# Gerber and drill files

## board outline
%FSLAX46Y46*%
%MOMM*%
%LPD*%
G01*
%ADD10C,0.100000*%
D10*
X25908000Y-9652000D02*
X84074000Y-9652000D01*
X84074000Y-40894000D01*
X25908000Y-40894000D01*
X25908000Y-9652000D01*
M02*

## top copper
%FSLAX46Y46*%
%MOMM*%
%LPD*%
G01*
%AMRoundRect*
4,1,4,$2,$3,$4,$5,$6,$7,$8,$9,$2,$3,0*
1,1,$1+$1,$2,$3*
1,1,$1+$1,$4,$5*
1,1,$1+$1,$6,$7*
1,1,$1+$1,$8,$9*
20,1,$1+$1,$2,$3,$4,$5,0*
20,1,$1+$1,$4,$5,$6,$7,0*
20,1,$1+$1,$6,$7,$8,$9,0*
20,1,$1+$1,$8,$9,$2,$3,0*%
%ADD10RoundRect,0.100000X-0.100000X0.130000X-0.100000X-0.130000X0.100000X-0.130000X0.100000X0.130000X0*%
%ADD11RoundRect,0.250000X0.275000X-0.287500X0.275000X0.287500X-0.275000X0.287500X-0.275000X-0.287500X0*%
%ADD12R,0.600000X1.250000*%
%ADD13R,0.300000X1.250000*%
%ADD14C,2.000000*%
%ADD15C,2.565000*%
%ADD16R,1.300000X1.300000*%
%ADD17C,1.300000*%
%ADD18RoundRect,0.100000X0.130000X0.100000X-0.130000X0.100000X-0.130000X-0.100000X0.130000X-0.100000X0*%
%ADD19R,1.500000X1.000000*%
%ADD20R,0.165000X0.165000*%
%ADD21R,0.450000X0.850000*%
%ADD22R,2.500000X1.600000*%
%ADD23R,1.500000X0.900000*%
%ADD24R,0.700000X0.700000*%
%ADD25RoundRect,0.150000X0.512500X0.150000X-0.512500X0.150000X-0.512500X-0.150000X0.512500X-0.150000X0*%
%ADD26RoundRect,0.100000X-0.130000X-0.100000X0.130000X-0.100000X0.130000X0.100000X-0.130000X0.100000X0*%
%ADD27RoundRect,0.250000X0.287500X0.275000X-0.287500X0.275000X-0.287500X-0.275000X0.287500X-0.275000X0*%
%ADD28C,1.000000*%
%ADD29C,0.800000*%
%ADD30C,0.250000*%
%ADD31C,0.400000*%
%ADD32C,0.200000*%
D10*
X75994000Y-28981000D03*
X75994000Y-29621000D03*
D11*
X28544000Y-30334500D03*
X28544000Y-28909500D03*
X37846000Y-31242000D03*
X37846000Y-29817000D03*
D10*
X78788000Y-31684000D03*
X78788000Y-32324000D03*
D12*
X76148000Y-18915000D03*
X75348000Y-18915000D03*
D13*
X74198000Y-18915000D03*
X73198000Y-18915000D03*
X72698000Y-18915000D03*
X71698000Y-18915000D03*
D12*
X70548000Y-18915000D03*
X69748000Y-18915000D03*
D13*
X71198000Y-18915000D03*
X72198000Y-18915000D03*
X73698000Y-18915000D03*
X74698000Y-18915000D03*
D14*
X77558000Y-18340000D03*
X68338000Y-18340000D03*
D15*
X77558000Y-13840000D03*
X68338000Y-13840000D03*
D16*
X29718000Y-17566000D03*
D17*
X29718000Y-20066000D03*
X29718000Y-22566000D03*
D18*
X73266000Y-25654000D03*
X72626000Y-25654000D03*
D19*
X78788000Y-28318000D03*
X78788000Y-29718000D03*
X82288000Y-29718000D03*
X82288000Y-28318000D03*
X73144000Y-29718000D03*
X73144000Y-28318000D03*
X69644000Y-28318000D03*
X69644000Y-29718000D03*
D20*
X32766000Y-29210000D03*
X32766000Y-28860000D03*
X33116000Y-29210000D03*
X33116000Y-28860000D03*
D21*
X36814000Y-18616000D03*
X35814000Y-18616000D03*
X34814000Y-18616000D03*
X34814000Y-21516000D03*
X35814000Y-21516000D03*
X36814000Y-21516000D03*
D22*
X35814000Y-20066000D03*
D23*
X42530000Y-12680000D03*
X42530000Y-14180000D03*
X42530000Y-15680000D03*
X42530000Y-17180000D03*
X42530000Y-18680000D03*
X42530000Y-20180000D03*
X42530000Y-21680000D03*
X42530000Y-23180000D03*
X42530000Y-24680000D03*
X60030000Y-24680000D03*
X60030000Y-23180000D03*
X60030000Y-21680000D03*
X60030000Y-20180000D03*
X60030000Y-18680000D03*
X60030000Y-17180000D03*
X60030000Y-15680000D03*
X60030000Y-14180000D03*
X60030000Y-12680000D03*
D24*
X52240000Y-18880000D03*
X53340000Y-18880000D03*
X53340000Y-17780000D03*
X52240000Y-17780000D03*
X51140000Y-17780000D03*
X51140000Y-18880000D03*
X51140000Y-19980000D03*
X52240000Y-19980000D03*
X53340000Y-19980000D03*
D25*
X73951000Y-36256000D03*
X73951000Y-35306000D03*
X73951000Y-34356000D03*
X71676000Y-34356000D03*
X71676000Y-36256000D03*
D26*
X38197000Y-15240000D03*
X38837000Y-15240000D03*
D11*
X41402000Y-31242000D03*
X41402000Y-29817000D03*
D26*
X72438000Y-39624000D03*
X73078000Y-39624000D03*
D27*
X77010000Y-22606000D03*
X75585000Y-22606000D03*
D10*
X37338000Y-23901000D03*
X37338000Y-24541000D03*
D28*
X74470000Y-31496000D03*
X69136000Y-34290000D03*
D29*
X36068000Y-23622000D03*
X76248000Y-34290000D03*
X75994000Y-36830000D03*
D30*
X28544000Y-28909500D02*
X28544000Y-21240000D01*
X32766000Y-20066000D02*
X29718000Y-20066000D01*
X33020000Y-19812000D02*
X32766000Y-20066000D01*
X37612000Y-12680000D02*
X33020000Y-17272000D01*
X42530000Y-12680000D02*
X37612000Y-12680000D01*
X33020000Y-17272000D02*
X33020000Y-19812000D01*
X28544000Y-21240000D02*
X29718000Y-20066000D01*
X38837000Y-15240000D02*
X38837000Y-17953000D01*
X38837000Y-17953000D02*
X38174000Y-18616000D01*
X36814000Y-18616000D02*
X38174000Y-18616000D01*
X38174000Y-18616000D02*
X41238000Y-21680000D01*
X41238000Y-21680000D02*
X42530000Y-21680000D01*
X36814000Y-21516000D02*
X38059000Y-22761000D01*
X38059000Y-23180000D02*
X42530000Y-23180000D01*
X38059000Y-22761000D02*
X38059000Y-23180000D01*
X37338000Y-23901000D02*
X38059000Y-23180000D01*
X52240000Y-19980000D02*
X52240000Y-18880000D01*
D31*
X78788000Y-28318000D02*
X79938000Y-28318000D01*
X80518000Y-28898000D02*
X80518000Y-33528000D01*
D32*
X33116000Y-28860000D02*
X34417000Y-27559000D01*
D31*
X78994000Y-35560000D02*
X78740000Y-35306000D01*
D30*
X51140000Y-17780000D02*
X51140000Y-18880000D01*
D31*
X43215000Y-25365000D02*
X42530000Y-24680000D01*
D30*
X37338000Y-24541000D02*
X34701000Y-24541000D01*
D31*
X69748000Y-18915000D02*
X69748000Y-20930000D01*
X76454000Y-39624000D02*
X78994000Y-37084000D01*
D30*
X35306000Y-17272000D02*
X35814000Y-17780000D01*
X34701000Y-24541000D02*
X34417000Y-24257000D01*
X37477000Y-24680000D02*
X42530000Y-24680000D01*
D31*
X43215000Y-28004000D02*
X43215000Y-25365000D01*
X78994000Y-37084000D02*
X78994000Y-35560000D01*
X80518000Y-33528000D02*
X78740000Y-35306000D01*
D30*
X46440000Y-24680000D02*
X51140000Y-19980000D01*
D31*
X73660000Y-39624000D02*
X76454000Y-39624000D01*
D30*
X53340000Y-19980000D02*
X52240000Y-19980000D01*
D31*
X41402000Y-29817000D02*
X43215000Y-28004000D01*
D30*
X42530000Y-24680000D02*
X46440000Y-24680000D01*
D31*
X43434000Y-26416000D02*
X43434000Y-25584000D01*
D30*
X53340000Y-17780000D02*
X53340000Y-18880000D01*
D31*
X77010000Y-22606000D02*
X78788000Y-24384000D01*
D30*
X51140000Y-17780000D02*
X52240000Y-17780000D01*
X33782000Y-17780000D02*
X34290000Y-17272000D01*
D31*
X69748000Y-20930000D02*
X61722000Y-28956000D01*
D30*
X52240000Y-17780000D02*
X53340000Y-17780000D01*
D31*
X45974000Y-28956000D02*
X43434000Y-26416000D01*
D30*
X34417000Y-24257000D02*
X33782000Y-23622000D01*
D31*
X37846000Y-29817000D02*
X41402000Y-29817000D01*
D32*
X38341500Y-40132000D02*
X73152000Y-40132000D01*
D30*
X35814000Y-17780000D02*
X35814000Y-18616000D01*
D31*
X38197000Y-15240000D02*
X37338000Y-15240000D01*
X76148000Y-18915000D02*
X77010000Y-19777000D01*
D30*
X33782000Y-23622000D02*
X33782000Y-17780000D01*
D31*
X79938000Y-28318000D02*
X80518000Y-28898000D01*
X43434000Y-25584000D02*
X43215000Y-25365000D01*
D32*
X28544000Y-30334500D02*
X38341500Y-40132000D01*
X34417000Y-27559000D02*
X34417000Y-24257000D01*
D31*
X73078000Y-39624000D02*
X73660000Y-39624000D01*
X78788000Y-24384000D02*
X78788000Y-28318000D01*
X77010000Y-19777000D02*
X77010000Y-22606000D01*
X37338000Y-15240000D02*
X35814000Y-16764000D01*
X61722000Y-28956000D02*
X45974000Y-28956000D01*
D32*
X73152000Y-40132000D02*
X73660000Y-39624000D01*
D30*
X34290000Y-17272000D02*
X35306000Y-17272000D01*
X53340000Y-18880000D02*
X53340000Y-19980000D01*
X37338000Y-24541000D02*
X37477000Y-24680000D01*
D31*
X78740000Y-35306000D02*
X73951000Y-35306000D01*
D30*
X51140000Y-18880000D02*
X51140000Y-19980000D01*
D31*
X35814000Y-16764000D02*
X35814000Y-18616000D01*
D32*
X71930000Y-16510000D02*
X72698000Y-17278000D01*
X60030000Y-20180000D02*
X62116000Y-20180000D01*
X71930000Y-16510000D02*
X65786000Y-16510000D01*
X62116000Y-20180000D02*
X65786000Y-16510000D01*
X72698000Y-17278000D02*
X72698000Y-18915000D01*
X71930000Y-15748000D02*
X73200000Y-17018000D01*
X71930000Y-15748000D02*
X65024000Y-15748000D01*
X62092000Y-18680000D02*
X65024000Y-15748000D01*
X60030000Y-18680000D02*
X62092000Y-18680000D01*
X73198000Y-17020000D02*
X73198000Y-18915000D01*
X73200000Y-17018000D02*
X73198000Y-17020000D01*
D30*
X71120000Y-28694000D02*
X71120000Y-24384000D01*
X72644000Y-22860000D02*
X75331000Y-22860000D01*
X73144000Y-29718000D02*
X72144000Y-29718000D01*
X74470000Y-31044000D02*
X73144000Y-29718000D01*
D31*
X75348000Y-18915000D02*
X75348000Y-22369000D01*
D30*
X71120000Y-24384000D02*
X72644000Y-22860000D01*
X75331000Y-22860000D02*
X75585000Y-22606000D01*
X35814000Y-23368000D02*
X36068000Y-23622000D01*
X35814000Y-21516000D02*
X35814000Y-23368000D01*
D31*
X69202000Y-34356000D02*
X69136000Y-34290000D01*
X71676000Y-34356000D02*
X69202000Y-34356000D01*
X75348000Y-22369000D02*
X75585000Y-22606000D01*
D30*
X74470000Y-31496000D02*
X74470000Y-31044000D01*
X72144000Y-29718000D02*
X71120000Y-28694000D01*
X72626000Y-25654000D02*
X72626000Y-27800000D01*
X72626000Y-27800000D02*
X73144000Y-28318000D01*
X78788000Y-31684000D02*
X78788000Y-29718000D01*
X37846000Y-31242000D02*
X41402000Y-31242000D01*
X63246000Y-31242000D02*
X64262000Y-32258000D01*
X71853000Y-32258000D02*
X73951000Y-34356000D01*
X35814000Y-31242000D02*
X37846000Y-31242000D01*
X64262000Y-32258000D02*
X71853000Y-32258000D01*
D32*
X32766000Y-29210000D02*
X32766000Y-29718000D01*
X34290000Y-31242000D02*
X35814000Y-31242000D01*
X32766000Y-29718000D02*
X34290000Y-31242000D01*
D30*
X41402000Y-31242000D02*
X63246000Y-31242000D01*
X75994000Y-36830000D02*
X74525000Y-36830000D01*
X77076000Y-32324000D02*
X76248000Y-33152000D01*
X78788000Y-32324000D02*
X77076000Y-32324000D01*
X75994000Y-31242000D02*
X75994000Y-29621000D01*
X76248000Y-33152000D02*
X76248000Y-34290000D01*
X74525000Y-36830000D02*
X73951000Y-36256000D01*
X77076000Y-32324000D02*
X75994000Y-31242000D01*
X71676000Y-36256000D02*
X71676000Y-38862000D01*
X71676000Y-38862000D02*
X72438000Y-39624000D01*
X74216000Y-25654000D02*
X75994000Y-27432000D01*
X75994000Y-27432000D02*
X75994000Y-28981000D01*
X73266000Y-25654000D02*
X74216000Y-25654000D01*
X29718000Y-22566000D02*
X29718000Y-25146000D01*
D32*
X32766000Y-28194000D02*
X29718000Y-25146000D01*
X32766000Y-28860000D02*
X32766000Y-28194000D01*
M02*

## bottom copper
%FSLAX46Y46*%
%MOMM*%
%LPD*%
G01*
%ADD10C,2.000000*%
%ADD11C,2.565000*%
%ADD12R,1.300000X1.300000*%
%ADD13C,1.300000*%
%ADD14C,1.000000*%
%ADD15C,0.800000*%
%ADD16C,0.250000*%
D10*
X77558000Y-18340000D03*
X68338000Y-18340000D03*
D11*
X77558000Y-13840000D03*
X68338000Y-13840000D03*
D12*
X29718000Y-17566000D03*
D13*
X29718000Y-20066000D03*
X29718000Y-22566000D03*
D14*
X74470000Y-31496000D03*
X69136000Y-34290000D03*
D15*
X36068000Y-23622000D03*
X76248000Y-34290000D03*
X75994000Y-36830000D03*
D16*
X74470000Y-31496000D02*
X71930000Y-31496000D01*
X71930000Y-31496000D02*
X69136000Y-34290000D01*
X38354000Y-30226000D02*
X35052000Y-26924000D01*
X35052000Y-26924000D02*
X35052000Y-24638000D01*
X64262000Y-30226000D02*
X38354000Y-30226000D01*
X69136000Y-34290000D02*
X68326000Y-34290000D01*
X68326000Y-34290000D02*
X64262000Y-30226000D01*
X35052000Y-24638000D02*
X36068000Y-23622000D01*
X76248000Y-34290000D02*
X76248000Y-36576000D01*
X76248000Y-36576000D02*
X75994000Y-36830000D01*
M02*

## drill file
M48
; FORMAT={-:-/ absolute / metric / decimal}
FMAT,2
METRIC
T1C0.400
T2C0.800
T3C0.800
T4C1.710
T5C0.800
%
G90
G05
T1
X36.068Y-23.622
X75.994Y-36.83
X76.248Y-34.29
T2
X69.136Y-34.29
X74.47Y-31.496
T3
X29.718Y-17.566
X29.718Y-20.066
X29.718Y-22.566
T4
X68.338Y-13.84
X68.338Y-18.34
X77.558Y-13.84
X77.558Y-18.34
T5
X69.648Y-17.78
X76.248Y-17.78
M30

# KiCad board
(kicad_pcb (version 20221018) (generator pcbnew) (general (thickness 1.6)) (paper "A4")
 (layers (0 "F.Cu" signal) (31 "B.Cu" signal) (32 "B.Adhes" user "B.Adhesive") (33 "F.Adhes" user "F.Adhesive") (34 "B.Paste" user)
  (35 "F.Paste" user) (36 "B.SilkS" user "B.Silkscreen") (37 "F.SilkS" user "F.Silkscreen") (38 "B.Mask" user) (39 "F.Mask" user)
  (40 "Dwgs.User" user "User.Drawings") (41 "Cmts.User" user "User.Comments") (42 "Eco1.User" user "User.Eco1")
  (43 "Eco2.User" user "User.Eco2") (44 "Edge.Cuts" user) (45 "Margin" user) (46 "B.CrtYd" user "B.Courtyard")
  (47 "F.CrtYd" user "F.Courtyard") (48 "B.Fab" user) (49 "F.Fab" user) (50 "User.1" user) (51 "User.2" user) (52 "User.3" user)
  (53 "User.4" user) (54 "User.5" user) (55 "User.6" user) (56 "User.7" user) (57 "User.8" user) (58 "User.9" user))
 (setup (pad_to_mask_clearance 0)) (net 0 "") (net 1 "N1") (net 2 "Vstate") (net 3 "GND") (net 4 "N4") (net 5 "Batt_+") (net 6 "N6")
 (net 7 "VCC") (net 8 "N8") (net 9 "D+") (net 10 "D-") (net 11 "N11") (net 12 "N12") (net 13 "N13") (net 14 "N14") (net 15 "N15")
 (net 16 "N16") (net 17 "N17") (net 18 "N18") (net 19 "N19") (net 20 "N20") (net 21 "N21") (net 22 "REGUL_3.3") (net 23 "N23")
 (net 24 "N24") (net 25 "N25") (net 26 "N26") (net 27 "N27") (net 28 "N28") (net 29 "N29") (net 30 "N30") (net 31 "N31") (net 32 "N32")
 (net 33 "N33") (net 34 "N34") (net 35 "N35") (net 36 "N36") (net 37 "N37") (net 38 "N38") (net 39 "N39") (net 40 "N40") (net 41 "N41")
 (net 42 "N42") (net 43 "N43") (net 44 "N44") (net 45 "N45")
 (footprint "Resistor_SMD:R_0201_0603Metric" (layer "F.Cu") (at 75.994 29.301 -90)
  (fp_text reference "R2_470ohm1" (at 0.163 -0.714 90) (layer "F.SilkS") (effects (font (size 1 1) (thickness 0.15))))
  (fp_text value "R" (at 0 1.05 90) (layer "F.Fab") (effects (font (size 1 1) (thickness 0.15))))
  (pad "" smd roundrect (at -0.345 0 270) (size 0.318 0.36) (layers "F.Paste") (roundrect_rratio 0.25))
  (pad "" smd roundrect (at 0.345 0 270) (size 0.318 0.36) (layers "F.Paste") (roundrect_rratio 0.25))
  (pad "1" smd roundrect (at -0.32 0 270) (size 0.46 0.4) (layers "F.Cu" "F.Mask") (roundrect_rratio 0.25) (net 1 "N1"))
  (pad "2" smd roundrect (at 0.32 0 270) (size 0.46 0.4) (layers "F.Cu" "F.Mask") (roundrect_rratio 0.25) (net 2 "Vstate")))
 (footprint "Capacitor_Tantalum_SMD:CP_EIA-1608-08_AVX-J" (layer "F.Cu") (at 28.544 29.622 90)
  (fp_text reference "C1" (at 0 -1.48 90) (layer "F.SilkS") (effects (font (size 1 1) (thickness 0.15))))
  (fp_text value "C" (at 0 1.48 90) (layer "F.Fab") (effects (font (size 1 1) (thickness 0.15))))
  (pad "1" smd roundrect (at -0.7125 0 90) (size 1.075 1.05) (layers "F.Cu" "F.Paste" "F.Mask") (roundrect_rratio 0.238095) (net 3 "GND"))
  (pad "2" smd roundrect (at 0.7125 0 90) (size 1.075 1.05) (layers "F.Cu" "F.Paste" "F.Mask") (roundrect_rratio 0.238095) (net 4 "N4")))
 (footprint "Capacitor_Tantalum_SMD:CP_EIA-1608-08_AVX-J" (layer "F.Cu") (at 37.846 30.5295 90)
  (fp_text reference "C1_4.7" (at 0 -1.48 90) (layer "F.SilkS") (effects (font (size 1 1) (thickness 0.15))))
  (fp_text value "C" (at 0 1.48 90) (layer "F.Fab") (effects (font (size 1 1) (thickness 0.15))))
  (pad "1" smd roundrect (at -0.7125 0 90) (size 1.075 1.05) (layers "F.Cu" "F.Paste" "F.Mask") (roundrect_rratio 0.238095) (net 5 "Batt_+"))
  (pad "2" smd roundrect (at 0.7125 0 90) (size 1.075 1.05) (layers "F.Cu" "F.Paste" "F.Mask") (roundrect_rratio 0.238095) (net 3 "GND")))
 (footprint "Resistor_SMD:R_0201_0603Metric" (layer "F.Cu") (at 78.788 32.004 -90)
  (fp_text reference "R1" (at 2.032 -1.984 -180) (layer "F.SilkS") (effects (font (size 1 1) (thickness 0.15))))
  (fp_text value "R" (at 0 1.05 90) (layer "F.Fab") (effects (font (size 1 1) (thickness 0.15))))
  (pad "" smd roundrect (at -0.345 0 270) (size 0.318 0.36) (layers "F.Paste") (roundrect_rratio 0.25))
  (pad "" smd roundrect (at 0.345 0 270) (size 0.318 0.36) (layers "F.Paste") (roundrect_rratio 0.25))
  (pad "1" smd roundrect (at -0.32 0 270) (size 0.46 0.4) (layers "F.Cu" "F.Mask") (roundrect_rratio 0.25) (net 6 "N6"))
  (pad "2" smd roundrect (at 0.32 0 270) (size 0.46 0.4) (layers "F.Cu" "F.Mask") (roundrect_rratio 0.25) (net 2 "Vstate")))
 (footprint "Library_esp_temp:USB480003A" (layer "F.Cu") (at 72.948 15.24 180)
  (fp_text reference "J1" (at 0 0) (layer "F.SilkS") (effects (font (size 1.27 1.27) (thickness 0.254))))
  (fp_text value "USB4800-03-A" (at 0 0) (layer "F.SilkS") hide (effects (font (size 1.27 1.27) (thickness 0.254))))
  (pad "" np_thru_hole circle (at -3.3 -2.54 180) (size 0.8 0.8) (drill 0.8) (layers "*.Cu" "*.Mask"))
  (pad "" np_thru_hole circle (at 3.3 -2.54 180) (size 0.8 0.8) (drill 0.8) (layers "*.Cu" "*.Mask"))
  (pad "A1" smd rect (at -3.2 -3.675 180) (size 0.6 1.25) (layers "F.Cu" "F.Paste" "F.Mask") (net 3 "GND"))
  (pad "A4" smd rect (at -2.4 -3.675 180) (size 0.6 1.25) (layers "F.Cu" "F.Paste" "F.Mask") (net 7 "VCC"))
  (pad "A5" smd rect (at -1.25 -3.675 180) (size 0.3 1.25) (layers "F.Cu" "F.Paste" "F.Mask") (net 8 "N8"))
  (pad "A6" smd rect (at -0.25 -3.675 180) (size 0.3 1.25) (layers "F.Cu" "F.Paste" "F.Mask") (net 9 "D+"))
  (pad "A7" smd rect (at 0.25 -3.675 180) (size 0.3 1.25) (layers "F.Cu" "F.Paste" "F.Mask") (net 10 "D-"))
  (pad "A8" smd rect (at 1.25 -3.675 180) (size 0.3 1.25) (layers "F.Cu" "F.Paste" "F.Mask") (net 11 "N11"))
  (pad "A9" smd rect (at 2.4 -3.675 180) (size 0.6 1.25) (layers "F.Cu" "F.Paste" "F.Mask") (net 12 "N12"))
  (pad "A12" smd rect (at 3.2 -3.675 180) (size 0.6 1.25) (layers "F.Cu" "F.Paste" "F.Mask") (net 3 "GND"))
  (pad "B5" smd rect (at 1.75 -3.675 180) (size 0.3 1.25) (layers "F.Cu" "F.Paste" "F.Mask") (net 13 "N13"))
  (pad "B6" smd rect (at 0.75 -3.675 180) (size 0.3 1.25) (layers "F.Cu" "F.Paste" "F.Mask") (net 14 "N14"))
  (pad "B7" smd rect (at -0.75 -3.675 180) (size 0.3 1.25) (layers "F.Cu" "F.Paste" "F.Mask") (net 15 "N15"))
  (pad "B8" smd rect (at -1.75 -3.675 180) (size 0.3 1.25) (layers "F.Cu" "F.Paste" "F.Mask") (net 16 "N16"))
  (pad "MH3" thru_hole circle (at -4.61 -3.1 180) (size 2 2) (drill 1.71) (layers "*.Cu" "*.Mask") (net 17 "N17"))
  (pad "MH4" thru_hole circle (at 4.61 -3.1 180) (size 2 2) (drill 1.71) (layers "*.Cu" "*.Mask") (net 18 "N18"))
  (pad "MH5" thru_hole circle (at -4.61 1.4 180) (size 2.565 2.565) (drill 1.71) (layers "*.Cu" "*.Mask") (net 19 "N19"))
  (pad "MH6" thru_hole circle (at 4.61 1.4 180) (size 2.565 2.565) (drill 1.71) (layers "*.Cu" "*.Mask") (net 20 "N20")))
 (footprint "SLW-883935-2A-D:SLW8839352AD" (layer "F.Cu") (at 29.718 17.566 -90)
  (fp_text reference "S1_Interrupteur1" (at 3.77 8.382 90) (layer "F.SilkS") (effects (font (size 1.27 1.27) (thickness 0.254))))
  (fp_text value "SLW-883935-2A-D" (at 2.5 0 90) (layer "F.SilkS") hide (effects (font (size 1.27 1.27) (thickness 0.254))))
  (pad "1" thru_hole rect (at 0 0 270) (size 1.3 1.3) (drill 0.8) (layers "*.Cu" "*.Mask") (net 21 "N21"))
  (pad "2" thru_hole circle (at 2.5 0 270) (size 1.3 1.3) (drill 0.8) (layers "*.Cu" "*.Mask") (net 4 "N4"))
  (pad "3" thru_hole circle (at 5 0 270) (size 1.3 1.3) (drill 0.8) (layers "*.Cu" "*.Mask") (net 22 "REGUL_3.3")))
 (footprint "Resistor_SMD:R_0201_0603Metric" (layer "F.Cu") (at 72.946 25.654 180)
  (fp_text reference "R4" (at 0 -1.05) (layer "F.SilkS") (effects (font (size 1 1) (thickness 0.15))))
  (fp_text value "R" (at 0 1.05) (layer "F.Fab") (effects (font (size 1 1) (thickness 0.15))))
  (pad "" smd roundrect (at -0.345 0 180) (size 0.318 0.36) (layers "F.Paste") (roundrect_rratio 0.25))
  (pad "" smd roundrect (at 0.345 0 180) (size 0.318 0.36) (layers "F.Paste") (roundrect_rratio 0.25))
  (pad "1" smd roundrect (at -0.32 0 180) (size 0.46 0.4) (layers "F.Cu" "F.Mask") (roundrect_rratio 0.25) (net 1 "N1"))
  (pad "2" smd roundrect (at 0.32 0 180) (size 0.46 0.4) (layers "F.Cu" "F.Mask") (roundrect_rratio 0.25) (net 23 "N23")))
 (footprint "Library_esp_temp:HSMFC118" (layer "F.Cu") (at 80.538 29.018 180)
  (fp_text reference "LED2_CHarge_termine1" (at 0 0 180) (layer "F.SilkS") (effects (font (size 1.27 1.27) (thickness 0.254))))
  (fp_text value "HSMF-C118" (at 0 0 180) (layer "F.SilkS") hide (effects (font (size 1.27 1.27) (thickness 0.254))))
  (pad "1" smd rect (at 1.75 0.7 270) (size 1 1.5) (layers "F.Cu" "F.Paste" "F.Mask") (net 3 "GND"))
  (pad "2" smd rect (at 1.75 -0.7 270) (size 1 1.5) (layers "F.Cu" "F.Paste" "F.Mask") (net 6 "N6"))
  (pad "3" smd rect (at -1.75 -0.7 270) (size 1 1.5) (layers "F.Cu" "F.Paste" "F.Mask") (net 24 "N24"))
  (pad "4" smd rect (at -1.75 0.7 270) (size 1 1.5) (layers "F.Cu" "F.Paste" "F.Mask") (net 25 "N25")))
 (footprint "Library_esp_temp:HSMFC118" (layer "F.Cu") (at 71.394 29.018)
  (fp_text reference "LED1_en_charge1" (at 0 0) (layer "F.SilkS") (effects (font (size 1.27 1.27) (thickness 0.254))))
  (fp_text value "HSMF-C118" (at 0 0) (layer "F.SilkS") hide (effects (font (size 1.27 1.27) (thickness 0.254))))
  (pad "1" smd rect (at 1.75 0.7 90) (size 1 1.5) (layers "F.Cu" "F.Paste" "F.Mask") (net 7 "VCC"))
  (pad "2" smd rect (at 1.75 -0.7 90) (size 1 1.5) (layers "F.Cu" "F.Paste" "F.Mask") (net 23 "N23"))
  (pad "3" smd rect (at -1.75 -0.7 90) (size 1 1.5) (layers "F.Cu" "F.Paste" "F.Mask") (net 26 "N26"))
  (pad "4" smd rect (at -1.75 0.7 90) (size 1 1.5) (layers "F.Cu" "F.Paste" "F.Mask") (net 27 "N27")))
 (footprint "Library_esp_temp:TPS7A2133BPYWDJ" (layer "F.Cu") (at 32.941 29.035 90)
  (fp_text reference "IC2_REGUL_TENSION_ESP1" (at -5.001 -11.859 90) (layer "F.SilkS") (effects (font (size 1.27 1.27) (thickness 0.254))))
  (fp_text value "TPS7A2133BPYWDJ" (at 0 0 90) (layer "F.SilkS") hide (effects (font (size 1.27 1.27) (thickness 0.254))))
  (pad "A1" smd rect (at -0.175 -0.175 180) (size 0.165 0.165) (layers "F.Cu" "F.Paste" "F.Mask") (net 5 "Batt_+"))
  (pad "A2" smd rect (at 0.175 -0.175 180) (size 0.165 0.165) (layers "F.Cu" "F.Paste" "F.Mask") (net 22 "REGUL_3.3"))
  (pad "B1" smd rect (at -0.175 0.175 180) (size 0.165 0.165) (layers "F.Cu" "F.Paste" "F.Mask") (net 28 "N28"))
  (pad "B2" smd rect (at 0.175 0.175 180) (size 0.165 0.165) (layers "F.Cu" "F.Paste" "F.Mask") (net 3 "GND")))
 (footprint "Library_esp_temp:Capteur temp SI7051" (layer "F.Cu") (at 35.814 20.066 -90)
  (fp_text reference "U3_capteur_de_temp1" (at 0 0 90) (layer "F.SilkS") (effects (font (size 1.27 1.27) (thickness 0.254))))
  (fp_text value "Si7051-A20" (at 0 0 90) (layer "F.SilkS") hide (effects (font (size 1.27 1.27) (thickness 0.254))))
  (pad "1" smd rect (at -1.45 -1) (size 0.45 0.85) (layers "F.Cu" "F.Paste" "F.Mask") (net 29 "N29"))
  (pad "2" smd rect (at -1.45 0) (size 0.45 0.85) (layers "F.Cu" "F.Paste" "F.Mask") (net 3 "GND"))
  (pad "3" smd rect (at -1.45 1) (size 0.45 0.85) (layers "F.Cu" "F.Paste" "F.Mask") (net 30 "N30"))
  (pad "4" smd rect (at 1.45 1) (size 0.45 0.85) (layers "F.Cu" "F.Paste" "F.Mask") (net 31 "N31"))
  (pad "5" smd rect (at 1.45 0) (size 0.45 0.85) (layers "F.Cu" "F.Paste" "F.Mask") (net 7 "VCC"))
  (pad "6" smd rect (at 1.45 -1) (size 0.45 0.85) (layers "F.Cu" "F.Paste" "F.Mask") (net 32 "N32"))
  (pad "7" smd rect (at 0 0 270) (size 1.6 2.5) (layers "F.Cu" "F.Paste" "F.Mask")))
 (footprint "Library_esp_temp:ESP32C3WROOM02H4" (layer "F.Cu") (at 41.78 25.58)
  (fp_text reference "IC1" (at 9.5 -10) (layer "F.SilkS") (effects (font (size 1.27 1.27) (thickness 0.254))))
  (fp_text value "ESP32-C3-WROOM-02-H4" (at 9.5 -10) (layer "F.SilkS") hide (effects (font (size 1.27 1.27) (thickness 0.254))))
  (pad "1" smd rect (at 0.75 -12.9 90) (size 0.9 1.5) (layers "F.Cu" "F.Paste" "F.Mask") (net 4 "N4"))
  (pad "2" smd rect (at 0.75 -11.4 90) (size 0.9 1.5) (layers "F.Cu" "F.Paste" "F.Mask") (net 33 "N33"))
  (pad "3" smd rect (at 0.75 -9.9 90) (size 0.9 1.5) (layers "F.Cu" "F.Paste" "F.Mask") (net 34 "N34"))
  (pad "4" smd rect (at 0.75 -8.4 90) (size 0.9 1.5) (layers "F.Cu" "F.Paste" "F.Mask") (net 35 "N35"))
  (pad "5" smd rect (at 0.75 -6.9 90) (size 0.9 1.5) (layers "F.Cu" "F.Paste" "F.Mask") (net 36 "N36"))
  (pad "6" smd rect (at 0.75 -5.4 90) (size 0.9 1.5) (layers "F.Cu" "F.Paste" "F.Mask") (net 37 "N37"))
  (pad "7" smd rect (at 0.75 -3.9 90) (size 0.9 1.5) (layers "F.Cu" "F.Paste" "F.Mask") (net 29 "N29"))
  (pad "8" smd rect (at 0.75 -2.4 90) (size 0.9 1.5) (layers "F.Cu" "F.Paste" "F.Mask") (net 32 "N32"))
  (pad "9" smd rect (at 0.75 -0.9 90) (size 0.9 1.5) (layers "F.Cu" "F.Paste" "F.Mask") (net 3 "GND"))
  (pad "10" smd rect (at 18.25 -0.9 90) (size 0.9 1.5) (layers "F.Cu" "F.Paste" "F.Mask") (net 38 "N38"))
  (pad "11" smd rect (at 18.25 -2.4 90) (size 0.9 1.5) (layers "F.Cu" "F.Paste" "F.Mask") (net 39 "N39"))
  (pad "12" smd rect (at 18.25 -3.9 90) (size 0.9 1.5) (layers "F.Cu" "F.Paste" "F.Mask") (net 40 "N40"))
  (pad "13" smd rect (at 18.25 -5.4 90) (size 0.9 1.5) (layers "F.Cu" "F.Paste" "F.Mask") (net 10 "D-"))
  (pad "14" smd rect (at 18.25 -6.9 90) (size 0.9 1.5) (layers "F.Cu" "F.Paste" "F.Mask") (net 9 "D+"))
  (pad "15" smd rect (at 18.25 -8.4 90) (size 0.9 1.5) (layers "F.Cu" "F.Paste" "F.Mask") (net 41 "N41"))
  (pad "16" smd rect (at 18.25 -9.9 90) (size 0.9 1.5) (layers "F.Cu" "F.Paste" "F.Mask") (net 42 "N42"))
  (pad "17" smd rect (at 18.25 -11.4 90) (size 0.9 1.5) (layers "F.Cu" "F.Paste" "F.Mask") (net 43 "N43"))
  (pad "18" smd rect (at 18.25 -12.9 90) (size 0.9 1.5) (layers "F.Cu" "F.Paste" "F.Mask") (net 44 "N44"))
  (pad "19" smd rect (at 10.46 -6.7 90) (size 0.7 0.7) (layers "F.Cu" "F.Paste" "F.Mask") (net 3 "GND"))
  (pad "20" smd rect (at 11.56 -6.7 90) (size 0.7 0.7) (layers "F.Cu" "F.Paste" "F.Mask") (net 3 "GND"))
  (pad "21" smd rect (at 11.56 -7.8 90) (size 0.7 0.7) (layers "F.Cu" "F.Paste" "F.Mask") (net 3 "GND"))
  (pad "22" smd rect (at 10.46 -7.8 90) (size 0.7 0.7) (layers "F.Cu" "F.Paste" "F.Mask") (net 3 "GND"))
  (pad "23" smd rect (at 9.36 -7.8 90) (size 0.7 0.7) (layers "F.Cu" "F.Paste" "F.Mask") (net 3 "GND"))
  (pad "24" smd rect (at 9.36 -6.7 90) (size 0.7 0.7) (layers "F.Cu" "F.Paste" "F.Mask") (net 3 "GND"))
  (pad "25" smd rect (at 9.36 -5.6 90) (size 0.7 0.7) (layers "F.Cu" "F.Paste" "F.Mask") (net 3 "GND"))
  (pad "26" smd rect (at 10.46 -5.6 90) (size 0.7 0.7) (layers "F.Cu" "F.Paste" "F.Mask") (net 3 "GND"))
  (pad "27" smd rect (at 11.56 -5.6 90) (size 0.7 0.7) (layers "F.Cu" "F.Paste" "F.Mask") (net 3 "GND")))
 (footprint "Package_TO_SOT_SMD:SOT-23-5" (layer "F.Cu") (at 72.8135 35.306 180)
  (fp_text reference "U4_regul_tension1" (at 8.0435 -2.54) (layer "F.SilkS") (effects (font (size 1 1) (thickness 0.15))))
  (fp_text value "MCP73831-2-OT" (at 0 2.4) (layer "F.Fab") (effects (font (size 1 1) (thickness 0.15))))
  (pad "1" smd roundrect (at -1.1375 -0.95 180) (size 1.325 0.6) (layers "F.Cu" "F.Paste" "F.Mask") (roundrect_rratio 0.25) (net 2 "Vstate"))
  (pad "2" smd roundrect (at -1.1375 0 180) (size 1.325 0.6) (layers "F.Cu" "F.Paste" "F.Mask") (roundrect_rratio 0.25) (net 3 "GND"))
  (pad "3" smd roundrect (at -1.1375 0.95 180) (size 1.325 0.6) (layers "F.Cu" "F.Paste" "F.Mask") (roundrect_rratio 0.25) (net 5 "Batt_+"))
  (pad "4" smd roundrect (at 1.1375 0.95 180) (size 1.325 0.6) (layers "F.Cu" "F.Paste" "F.Mask") (roundrect_rratio 0.25) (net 7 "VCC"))
  (pad "5" smd roundrect (at 1.1375 -0.95 180) (size 1.325 0.6) (layers "F.Cu" "F.Paste" "F.Mask") (roundrect_rratio 0.25) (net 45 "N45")))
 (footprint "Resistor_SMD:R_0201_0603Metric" (layer "F.Cu") (at 38.517 15.24)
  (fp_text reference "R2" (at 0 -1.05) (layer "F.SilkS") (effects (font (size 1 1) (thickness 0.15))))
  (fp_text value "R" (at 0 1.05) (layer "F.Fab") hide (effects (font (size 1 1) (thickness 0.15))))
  (pad "" smd roundrect (at -0.345 0) (size 0.318 0.36) (layers "F.Paste") (roundrect_rratio 0.25))
  (pad "" smd roundrect (at 0.345 0) (size 0.318 0.36) (layers "F.Paste") (roundrect_rratio 0.25))
  (pad "1" smd roundrect (at -0.32 0) (size 0.46 0.4) (layers "F.Cu" "F.Mask") (roundrect_rratio 0.25) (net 3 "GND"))
  (pad "2" smd roundrect (at 0.32 0) (size 0.46 0.4) (layers "F.Cu" "F.Mask") (roundrect_rratio 0.25) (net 29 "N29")))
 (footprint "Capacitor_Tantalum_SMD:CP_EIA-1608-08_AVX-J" (layer "F.Cu") (at 41.402 30.5295 90)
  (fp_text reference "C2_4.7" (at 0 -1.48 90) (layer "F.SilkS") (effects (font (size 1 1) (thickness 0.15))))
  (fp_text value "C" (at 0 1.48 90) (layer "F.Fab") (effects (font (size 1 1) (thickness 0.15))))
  (pad "1" smd roundrect (at -0.7125 0 90) (size 1.075 1.05) (layers "F.Cu" "F.Paste" "F.Mask") (roundrect_rratio 0.238095) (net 5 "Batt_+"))
  (pad "2" smd roundrect (at 0.7125 0 90) (size 1.075 1.05) (layers "F.Cu" "F.Paste" "F.Mask") (roundrect_rratio 0.238095) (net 3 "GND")))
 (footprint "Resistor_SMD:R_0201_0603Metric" (layer "F.Cu") (at 72.758 39.624)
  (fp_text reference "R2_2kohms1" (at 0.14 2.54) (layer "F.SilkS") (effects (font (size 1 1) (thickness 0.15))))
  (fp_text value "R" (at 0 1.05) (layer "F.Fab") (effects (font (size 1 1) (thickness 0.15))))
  (pad "" smd roundrect (at -0.345 0) (size 0.318 0.36) (layers "F.Paste") (roundrect_rratio 0.25))
  (pad "" smd roundrect (at 0.345 0) (size 0.318 0.36) (layers "F.Paste") (roundrect_rratio 0.25))
  (pad "1" smd roundrect (at -0.32 0) (size 0.46 0.4) (layers "F.Cu" "F.Mask") (roundrect_rratio 0.25) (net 45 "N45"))
  (pad "2" smd roundrect (at 0.32 0) (size 0.46 0.4) (layers "F.Cu" "F.Mask") (roundrect_rratio 0.25) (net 3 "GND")))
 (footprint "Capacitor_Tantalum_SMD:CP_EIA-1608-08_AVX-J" (layer "F.Cu") (at 76.2975 22.606 180)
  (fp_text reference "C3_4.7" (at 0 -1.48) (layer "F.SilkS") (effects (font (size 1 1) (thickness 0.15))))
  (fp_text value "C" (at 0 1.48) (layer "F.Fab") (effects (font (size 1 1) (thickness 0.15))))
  (pad "1" smd roundrect (at -0.7125 0 180) (size 1.075 1.05) (layers "F.Cu" "F.Paste" "F.Mask") (roundrect_rratio 0.238095) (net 3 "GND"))
  (pad "2" smd roundrect (at 0.7125 0 180) (size 1.075 1.05) (layers "F.Cu" "F.Paste" "F.Mask") (roundrect_rratio 0.238095) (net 7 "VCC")))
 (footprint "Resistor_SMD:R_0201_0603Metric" (layer "F.Cu") (at 37.338 24.221 -90)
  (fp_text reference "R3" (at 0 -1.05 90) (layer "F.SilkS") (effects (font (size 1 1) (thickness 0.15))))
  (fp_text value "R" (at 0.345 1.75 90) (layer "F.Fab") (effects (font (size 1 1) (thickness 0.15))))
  (pad "" smd roundrect (at -0.345 0 270) (size 0.318 0.36) (layers "F.Paste") (roundrect_rratio 0.25))
  (pad "" smd roundrect (at 0.345 0 270) (size 0.318 0.36) (layers "F.Paste") (roundrect_rratio 0.25))
  (pad "1" smd roundrect (at -0.32 0 270) (size 0.46 0.4) (layers "F.Cu" "F.Mask") (roundrect_rratio 0.25) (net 32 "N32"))
  (pad "2" smd roundrect (at 0.32 0 270) (size 0.46 0.4) (layers "F.Cu" "F.Mask") (roundrect_rratio 0.25) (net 3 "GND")))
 (gr_rect (start 25.908 9.652) (end 84.074 40.894) (stroke (width 0.1) (type default)) (fill none) (layer "Edge.Cuts"))
 (segment (start 28.544 28.9095) (end 28.544 21.24) (width 0.25) (layer "F.Cu") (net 4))
 (segment (start 32.766 20.066) (end 29.718 20.066) (width 0.25) (layer "F.Cu") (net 4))
 (segment (start 33.02 19.812) (end 32.766 20.066) (width 0.25) (layer "F.Cu") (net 4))
 (segment (start 37.612 12.68) (end 33.02 17.272) (width 0.25) (layer "F.Cu") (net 4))
 (segment (start 42.53 12.68) (end 37.612 12.68) (width 0.25) (layer "F.Cu") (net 4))
 (segment (start 33.02 17.272) (end 33.02 19.812) (width 0.25) (layer "F.Cu") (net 4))
 (segment (start 28.544 21.24) (end 29.718 20.066) (width 0.25) (layer "F.Cu") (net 4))
 (segment (start 38.837 15.24) (end 38.837 17.953) (width 0.25) (layer "F.Cu") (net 29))
 (segment (start 38.837 17.953) (end 38.174 18.616) (width 0.25) (layer "F.Cu") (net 29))
 (segment (start 36.814 18.616) (end 38.174 18.616) (width 0.25) (layer "F.Cu") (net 29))
 (segment (start 38.174 18.616) (end 41.238 21.68) (width 0.25) (layer "F.Cu") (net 29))
 (segment (start 41.238 21.68) (end 42.53 21.68) (width 0.25) (layer "F.Cu") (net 29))
 (segment (start 36.814 21.516) (end 38.059 22.761) (width 0.25) (layer "F.Cu") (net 32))
 (segment (start 38.059 23.18) (end 42.53 23.18) (width 0.25) (layer "F.Cu") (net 32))
 (segment (start 38.059 22.761) (end 38.059 23.18) (width 0.25) (layer "F.Cu") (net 32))
 (segment (start 37.338 23.901) (end 38.059 23.18) (width 0.25) (layer "F.Cu") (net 32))
 (segment (start 52.24 19.98) (end 52.24 18.88) (width 0.25) (layer "F.Cu") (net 3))
 (segment (start 78.788 28.318) (end 79.938 28.318) (width 0.4) (layer "F.Cu") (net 3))
 (segment (start 80.518 28.898) (end 80.518 33.528) (width 0.4) (layer "F.Cu") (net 3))
 (segment (start 33.116 28.86) (end 34.417 27.559) (width 0.2) (layer "F.Cu") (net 3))
 (segment (start 78.994 35.56) (end 78.74 35.306) (width 0.4) (layer "F.Cu") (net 3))
 (segment (start 51.14 17.78) (end 51.14 18.88) (width 0.25) (layer "F.Cu") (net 3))
 (segment (start 43.215 25.365) (end 42.53 24.68) (width 0.4) (layer "F.Cu") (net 3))
 (segment (start 37.338 24.541) (end 34.701 24.541) (width 0.25) (layer "F.Cu") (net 3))
 (segment (start 69.748 18.915) (end 69.748 20.93) (width 0.4) (layer "F.Cu") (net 3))
 (segment (start 76.454 39.624) (end 78.994 37.084) (width 0.4) (layer "F.Cu") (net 3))
 (segment (start 35.306 17.272) (end 35.814 17.78) (width 0.25) (layer "F.Cu") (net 3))
 (segment (start 34.701 24.541) (end 34.417 24.257) (width 0.25) (layer "F.Cu") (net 3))
 (segment (start 37.477 24.68) (end 42.53 24.68) (width 0.25) (layer "F.Cu") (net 3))
 (segment (start 43.215 28.004) (end 43.215 25.365) (width 0.4) (layer "F.Cu") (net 3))
 (segment (start 78.994 37.084) (end 78.994 35.56) (width 0.4) (layer "F.Cu") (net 3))
 (segment (start 80.518 33.528) (end 78.74 35.306) (width 0.4) (layer "F.Cu") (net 3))
 (segment (start 46.44 24.68) (end 51.14 19.98) (width 0.25) (layer "F.Cu") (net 3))
 (segment (start 73.66 39.624) (end 76.454 39.624) (width 0.4) (layer "F.Cu") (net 3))
 (segment (start 53.34 19.98) (end 52.24 19.98) (width 0.25) (layer "F.Cu") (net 3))
 (segment (start 41.402 29.817) (end 43.215 28.004) (width 0.4) (layer "F.Cu") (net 3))
 (segment (start 42.53 24.68) (end 46.44 24.68) (width 0.25) (layer "F.Cu") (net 3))
 (segment (start 43.434 26.416) (end 43.434 25.584) (width 0.4) (layer "F.Cu") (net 3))
 (segment (start 53.34 17.78) (end 53.34 18.88) (width 0.25) (layer "F.Cu") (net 3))
 (segment (start 77.01 22.606) (end 78.788 24.384) (width 0.4) (layer "F.Cu") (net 3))
 (segment (start 51.14 17.78) (end 52.24 17.78) (width 0.25) (layer "F.Cu") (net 3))
 (segment (start 33.782 17.78) (end 34.29 17.272) (width 0.25) (layer "F.Cu") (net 3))
 (segment (start 69.748 20.93) (end 61.722 28.956) (width 0.4) (layer "F.Cu") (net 3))
 (segment (start 52.24 17.78) (end 53.34 17.78) (width 0.25) (layer "F.Cu") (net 3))
 (segment (start 45.974 28.956) (end 43.434 26.416) (width 0.4) (layer "F.Cu") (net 3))
 (segment (start 34.417 24.257) (end 33.782 23.622) (width 0.25) (layer "F.Cu") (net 3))
 (segment (start 37.846 29.817) (end 41.402 29.817) (width 0.4) (layer "F.Cu") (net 3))
 (segment (start 38.3415 40.132) (end 73.152 40.132) (width 0.2) (layer "F.Cu") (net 3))
 (segment (start 35.814 17.78) (end 35.814 18.616) (width 0.25) (layer "F.Cu") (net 3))
 (segment (start 38.197 15.24) (end 37.338 15.24) (width 0.4) (layer "F.Cu") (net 3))
 (segment (start 76.148 18.915) (end 77.01 19.777) (width 0.4) (layer "F.Cu") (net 3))
 (segment (start 33.782 23.622) (end 33.782 17.78) (width 0.25) (layer "F.Cu") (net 3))
 (segment (start 79.938 28.318) (end 80.518 28.898) (width 0.4) (layer "F.Cu") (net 3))
 (segment (start 43.434 25.584) (end 43.215 25.365) (width 0.4) (layer "F.Cu") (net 3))
 (segment (start 28.544 30.3345) (end 38.3415 40.132) (width 0.2) (layer "F.Cu") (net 3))
 (segment (start 34.417 27.559) (end 34.417 24.257) (width 0.2) (layer "F.Cu") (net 3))
 (segment (start 73.078 39.624) (end 73.66 39.624) (width 0.4) (layer "F.Cu") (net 3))
 (segment (start 78.788 24.384) (end 78.788 28.318) (width 0.4) (layer "F.Cu") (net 3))
 (segment (start 77.01 19.777) (end 77.01 22.606) (width 0.4) (layer "F.Cu") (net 3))
 (segment (start 37.338 15.24) (end 35.814 16.764) (width 0.4) (layer "F.Cu") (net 3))
 (segment (start 61.722 28.956) (end 45.974 28.956) (width 0.4) (layer "F.Cu") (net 3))
 (segment (start 73.152 40.132) (end 73.66 39.624) (width 0.2) (layer "F.Cu") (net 3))
 (segment (start 34.29 17.272) (end 35.306 17.272) (width 0.25) (layer "F.Cu") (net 3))
 (segment (start 53.34 18.88) (end 53.34 19.98) (width 0.25) (layer "F.Cu") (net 3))
 (segment (start 37.338 24.541) (end 37.477 24.68) (width 0.25) (layer "F.Cu") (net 3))
 (segment (start 78.74 35.306) (end 73.951 35.306) (width 0.4) (layer "F.Cu") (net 3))
 (segment (start 51.14 18.88) (end 51.14 19.98) (width 0.25) (layer "F.Cu") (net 3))
 (segment (start 35.814 16.764) (end 35.814 18.616) (width 0.4) (layer "F.Cu") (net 3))
 (segment (start 71.93 16.51) (end 72.698 17.278) (width 0.2) (layer "F.Cu") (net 10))
 (segment (start 60.03 20.18) (end 62.116 20.18) (width 0.2) (layer "F.Cu") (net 10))
 (segment (start 71.93 16.51) (end 65.786 16.51) (width 0.2) (layer "F.Cu") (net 10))
 (segment (start 62.116 20.18) (end 65.786 16.51) (width 0.2) (layer "F.Cu") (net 10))
 (segment (start 72.698 17.278) (end 72.698 18.915) (width 0.2) (layer "F.Cu") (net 10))
 (segment (start 71.93 15.748) (end 73.2 17.018) (width 0.2) (layer "F.Cu") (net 9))
 (segment (start 71.93 15.748) (end 65.024 15.748) (width 0.2) (layer "F.Cu") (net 9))
 (segment (start 62.092 18.68) (end 65.024 15.748) (width 0.2) (layer "F.Cu") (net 9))
 (segment (start 60.03 18.68) (end 62.092 18.68) (width 0.2) (layer "F.Cu") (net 9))
 (segment (start 73.198 17.02) (end 73.198 18.915) (width 0.2) (layer "F.Cu") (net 9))
 (segment (start 73.2 17.018) (end 73.198 17.02) (width 0.2) (layer "F.Cu") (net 9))
 (segment (start 71.12 28.694) (end 71.12 24.384) (width 0.25) (layer "F.Cu") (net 7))
 (segment (start 72.644 22.86) (end 75.331 22.86) (width 0.25) (layer "F.Cu") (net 7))
 (segment (start 73.144 29.718) (end 72.144 29.718) (width 0.25) (layer "F.Cu") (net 7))
 (segment (start 74.47 31.044) (end 73.144 29.718) (width 0.25) (layer "F.Cu") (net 7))
 (segment (start 75.348 18.915) (end 75.348 22.369) (width 0.4) (layer "F.Cu") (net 7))
 (segment (start 71.12 24.384) (end 72.644 22.86) (width 0.25) (layer "F.Cu") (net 7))
 (segment (start 75.331 22.86) (end 75.585 22.606) (width 0.25) (layer "F.Cu") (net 7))
 (segment (start 35.814 23.368) (end 36.068 23.622) (width 0.25) (layer "F.Cu") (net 7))
 (segment (start 35.814 21.516) (end 35.814 23.368) (width 0.25) (layer "F.Cu") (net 7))
 (segment (start 69.202 34.356) (end 69.136 34.29) (width 0.4) (layer "F.Cu") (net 7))
 (segment (start 71.676 34.356) (end 69.202 34.356) (width 0.4) (layer "F.Cu") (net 7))
 (segment (start 75.348 22.369) (end 75.585 22.606) (width 0.4) (layer "F.Cu") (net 7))
 (segment (start 74.47 31.496) (end 74.47 31.044) (width 0.25) (layer "F.Cu") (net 7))
 (segment (start 72.144 29.718) (end 71.12 28.694) (width 0.25) (layer "F.Cu") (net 7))
 (via (at 74.47 31.496) (size 1) (drill 0.8) (layers "F.Cu" "B.Cu") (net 7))
 (via (at 69.136 34.29) (size 1) (drill 0.8) (layers "F.Cu" "B.Cu") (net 7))
 (via (at 36.068 23.622) (size 0.8) (drill 0.4) (layers "F.Cu" "B.Cu") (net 7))
 (segment (start 74.47 31.496) (end 71.93 31.496) (width 0.25) (layer "B.Cu") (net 7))
 (segment (start 71.93 31.496) (end 69.136 34.29) (width 0.25) (layer "B.Cu") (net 7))
 (segment (start 38.354 30.226) (end 35.052 26.924) (width 0.25) (layer "B.Cu") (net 7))
 (segment (start 35.052 26.924) (end 35.052 24.638) (width 0.25) (layer "B.Cu") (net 7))
 (segment (start 64.262 30.226) (end 38.354 30.226) (width 0.25) (layer "B.Cu") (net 7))
 (segment (start 69.136 34.29) (end 68.326 34.29) (width 0.25) (layer "B.Cu") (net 7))
 (segment (start 68.326 34.29) (end 64.262 30.226) (width 0.25) (layer "B.Cu") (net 7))
 (segment (start 35.052 24.638) (end 36.068 23.622) (width 0.25) (layer "B.Cu") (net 7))
 (segment (start 72.626 25.654) (end 72.626 27.8) (width 0.25) (layer "F.Cu") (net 23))
 (segment (start 72.626 27.8) (end 73.144 28.318) (width 0.25) (layer "F.Cu") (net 23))
 (segment (start 78.788 31.684) (end 78.788 29.718) (width 0.25) (layer "F.Cu") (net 6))
 (segment (start 37.846 31.242) (end 41.402 31.242) (width 0.25) (layer "F.Cu") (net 5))
 (segment (start 63.246 31.242) (end 64.262 32.258) (width 0.25) (layer "F.Cu") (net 5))
 (segment (start 71.853 32.258) (end 73.951 34.356) (width 0.25) (layer "F.Cu") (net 5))
 (segment (start 35.814 31.242) (end 37.846 31.242) (width 0.25) (layer "F.Cu") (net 5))
 (segment (start 64.262 32.258) (end 71.853 32.258) (width 0.25) (layer "F.Cu") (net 5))
 (segment (start 32.766 29.21) (end 32.766 29.718) (width 0.2) (layer "F.Cu") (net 5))
 (segment (start 34.29 31.242) (end 35.814 31.242) (width 0.2) (layer "F.Cu") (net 5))
 (segment (start 32.766 29.718) (end 34.29 31.242) (width 0.2) (layer "F.Cu") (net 5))
 (segment (start 41.402 31.242) (end 63.246 31.242) (width 0.25) (layer "F.Cu") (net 5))
 (segment (start 75.994 36.83) (end 74.525 36.83) (width 0.25) (layer "F.Cu") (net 2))
 (segment (start 77.076 32.324) (end 76.248 33.152) (width 0.25) (layer "F.Cu") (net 2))
 (segment (start 78.788 32.324) (end 77.076 32.324) (width 0.25) (layer "F.Cu") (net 2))
 (segment (start 75.994 31.242) (end 75.994 29.621) (width 0.25) (layer "F.Cu") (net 2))
 (segment (start 76.248 33.152) (end 76.248 34.29) (width 0.25) (layer "F.Cu") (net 2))
 (segment (start 74.525 36.83) (end 73.951 36.256) (width 0.25) (layer "F.Cu") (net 2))
 (segment (start 77.076 32.324) (end 75.994 31.242) (width 0.25) (layer "F.Cu") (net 2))
 (via (at 76.248 34.29) (size 0.8) (drill 0.4) (layers "F.Cu" "B.Cu") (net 2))
 (via (at 75.994 36.83) (size 0.8) (drill 0.4) (layers "F.Cu" "B.Cu") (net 2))
 (segment (start 76.248 34.29) (end 76.248 36.576) (width 0.25) (layer "B.Cu") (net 2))
 (segment (start 76.248 36.576) (end 75.994 36.83) (width 0.25) (layer "B.Cu") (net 2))
 (segment (start 71.676 36.256) (end 71.676 38.862) (width 0.25) (layer "F.Cu") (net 45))
 (segment (start 71.676 38.862) (end 72.438 39.624) (width 0.25) (layer "F.Cu") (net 45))
 (segment (start 74.216 25.654) (end 75.994 27.432) (width 0.25) (layer "F.Cu") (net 1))
 (segment (start 75.994 27.432) (end 75.994 28.981) (width 0.25) (layer "F.Cu") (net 1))
 (segment (start 73.266 25.654) (end 74.216 25.654) (width 0.25) (layer "F.Cu") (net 1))
 (segment (start 29.718 22.566) (end 29.718 25.146) (width 0.25) (layer "F.Cu") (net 22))
 (segment (start 32.766 28.194) (end 29.718 25.146) (width 0.2) (layer "F.Cu") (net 22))
 (segment (start 32.766 28.86) (end 32.766 28.194) (width 0.2) (layer "F.Cu") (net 22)))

